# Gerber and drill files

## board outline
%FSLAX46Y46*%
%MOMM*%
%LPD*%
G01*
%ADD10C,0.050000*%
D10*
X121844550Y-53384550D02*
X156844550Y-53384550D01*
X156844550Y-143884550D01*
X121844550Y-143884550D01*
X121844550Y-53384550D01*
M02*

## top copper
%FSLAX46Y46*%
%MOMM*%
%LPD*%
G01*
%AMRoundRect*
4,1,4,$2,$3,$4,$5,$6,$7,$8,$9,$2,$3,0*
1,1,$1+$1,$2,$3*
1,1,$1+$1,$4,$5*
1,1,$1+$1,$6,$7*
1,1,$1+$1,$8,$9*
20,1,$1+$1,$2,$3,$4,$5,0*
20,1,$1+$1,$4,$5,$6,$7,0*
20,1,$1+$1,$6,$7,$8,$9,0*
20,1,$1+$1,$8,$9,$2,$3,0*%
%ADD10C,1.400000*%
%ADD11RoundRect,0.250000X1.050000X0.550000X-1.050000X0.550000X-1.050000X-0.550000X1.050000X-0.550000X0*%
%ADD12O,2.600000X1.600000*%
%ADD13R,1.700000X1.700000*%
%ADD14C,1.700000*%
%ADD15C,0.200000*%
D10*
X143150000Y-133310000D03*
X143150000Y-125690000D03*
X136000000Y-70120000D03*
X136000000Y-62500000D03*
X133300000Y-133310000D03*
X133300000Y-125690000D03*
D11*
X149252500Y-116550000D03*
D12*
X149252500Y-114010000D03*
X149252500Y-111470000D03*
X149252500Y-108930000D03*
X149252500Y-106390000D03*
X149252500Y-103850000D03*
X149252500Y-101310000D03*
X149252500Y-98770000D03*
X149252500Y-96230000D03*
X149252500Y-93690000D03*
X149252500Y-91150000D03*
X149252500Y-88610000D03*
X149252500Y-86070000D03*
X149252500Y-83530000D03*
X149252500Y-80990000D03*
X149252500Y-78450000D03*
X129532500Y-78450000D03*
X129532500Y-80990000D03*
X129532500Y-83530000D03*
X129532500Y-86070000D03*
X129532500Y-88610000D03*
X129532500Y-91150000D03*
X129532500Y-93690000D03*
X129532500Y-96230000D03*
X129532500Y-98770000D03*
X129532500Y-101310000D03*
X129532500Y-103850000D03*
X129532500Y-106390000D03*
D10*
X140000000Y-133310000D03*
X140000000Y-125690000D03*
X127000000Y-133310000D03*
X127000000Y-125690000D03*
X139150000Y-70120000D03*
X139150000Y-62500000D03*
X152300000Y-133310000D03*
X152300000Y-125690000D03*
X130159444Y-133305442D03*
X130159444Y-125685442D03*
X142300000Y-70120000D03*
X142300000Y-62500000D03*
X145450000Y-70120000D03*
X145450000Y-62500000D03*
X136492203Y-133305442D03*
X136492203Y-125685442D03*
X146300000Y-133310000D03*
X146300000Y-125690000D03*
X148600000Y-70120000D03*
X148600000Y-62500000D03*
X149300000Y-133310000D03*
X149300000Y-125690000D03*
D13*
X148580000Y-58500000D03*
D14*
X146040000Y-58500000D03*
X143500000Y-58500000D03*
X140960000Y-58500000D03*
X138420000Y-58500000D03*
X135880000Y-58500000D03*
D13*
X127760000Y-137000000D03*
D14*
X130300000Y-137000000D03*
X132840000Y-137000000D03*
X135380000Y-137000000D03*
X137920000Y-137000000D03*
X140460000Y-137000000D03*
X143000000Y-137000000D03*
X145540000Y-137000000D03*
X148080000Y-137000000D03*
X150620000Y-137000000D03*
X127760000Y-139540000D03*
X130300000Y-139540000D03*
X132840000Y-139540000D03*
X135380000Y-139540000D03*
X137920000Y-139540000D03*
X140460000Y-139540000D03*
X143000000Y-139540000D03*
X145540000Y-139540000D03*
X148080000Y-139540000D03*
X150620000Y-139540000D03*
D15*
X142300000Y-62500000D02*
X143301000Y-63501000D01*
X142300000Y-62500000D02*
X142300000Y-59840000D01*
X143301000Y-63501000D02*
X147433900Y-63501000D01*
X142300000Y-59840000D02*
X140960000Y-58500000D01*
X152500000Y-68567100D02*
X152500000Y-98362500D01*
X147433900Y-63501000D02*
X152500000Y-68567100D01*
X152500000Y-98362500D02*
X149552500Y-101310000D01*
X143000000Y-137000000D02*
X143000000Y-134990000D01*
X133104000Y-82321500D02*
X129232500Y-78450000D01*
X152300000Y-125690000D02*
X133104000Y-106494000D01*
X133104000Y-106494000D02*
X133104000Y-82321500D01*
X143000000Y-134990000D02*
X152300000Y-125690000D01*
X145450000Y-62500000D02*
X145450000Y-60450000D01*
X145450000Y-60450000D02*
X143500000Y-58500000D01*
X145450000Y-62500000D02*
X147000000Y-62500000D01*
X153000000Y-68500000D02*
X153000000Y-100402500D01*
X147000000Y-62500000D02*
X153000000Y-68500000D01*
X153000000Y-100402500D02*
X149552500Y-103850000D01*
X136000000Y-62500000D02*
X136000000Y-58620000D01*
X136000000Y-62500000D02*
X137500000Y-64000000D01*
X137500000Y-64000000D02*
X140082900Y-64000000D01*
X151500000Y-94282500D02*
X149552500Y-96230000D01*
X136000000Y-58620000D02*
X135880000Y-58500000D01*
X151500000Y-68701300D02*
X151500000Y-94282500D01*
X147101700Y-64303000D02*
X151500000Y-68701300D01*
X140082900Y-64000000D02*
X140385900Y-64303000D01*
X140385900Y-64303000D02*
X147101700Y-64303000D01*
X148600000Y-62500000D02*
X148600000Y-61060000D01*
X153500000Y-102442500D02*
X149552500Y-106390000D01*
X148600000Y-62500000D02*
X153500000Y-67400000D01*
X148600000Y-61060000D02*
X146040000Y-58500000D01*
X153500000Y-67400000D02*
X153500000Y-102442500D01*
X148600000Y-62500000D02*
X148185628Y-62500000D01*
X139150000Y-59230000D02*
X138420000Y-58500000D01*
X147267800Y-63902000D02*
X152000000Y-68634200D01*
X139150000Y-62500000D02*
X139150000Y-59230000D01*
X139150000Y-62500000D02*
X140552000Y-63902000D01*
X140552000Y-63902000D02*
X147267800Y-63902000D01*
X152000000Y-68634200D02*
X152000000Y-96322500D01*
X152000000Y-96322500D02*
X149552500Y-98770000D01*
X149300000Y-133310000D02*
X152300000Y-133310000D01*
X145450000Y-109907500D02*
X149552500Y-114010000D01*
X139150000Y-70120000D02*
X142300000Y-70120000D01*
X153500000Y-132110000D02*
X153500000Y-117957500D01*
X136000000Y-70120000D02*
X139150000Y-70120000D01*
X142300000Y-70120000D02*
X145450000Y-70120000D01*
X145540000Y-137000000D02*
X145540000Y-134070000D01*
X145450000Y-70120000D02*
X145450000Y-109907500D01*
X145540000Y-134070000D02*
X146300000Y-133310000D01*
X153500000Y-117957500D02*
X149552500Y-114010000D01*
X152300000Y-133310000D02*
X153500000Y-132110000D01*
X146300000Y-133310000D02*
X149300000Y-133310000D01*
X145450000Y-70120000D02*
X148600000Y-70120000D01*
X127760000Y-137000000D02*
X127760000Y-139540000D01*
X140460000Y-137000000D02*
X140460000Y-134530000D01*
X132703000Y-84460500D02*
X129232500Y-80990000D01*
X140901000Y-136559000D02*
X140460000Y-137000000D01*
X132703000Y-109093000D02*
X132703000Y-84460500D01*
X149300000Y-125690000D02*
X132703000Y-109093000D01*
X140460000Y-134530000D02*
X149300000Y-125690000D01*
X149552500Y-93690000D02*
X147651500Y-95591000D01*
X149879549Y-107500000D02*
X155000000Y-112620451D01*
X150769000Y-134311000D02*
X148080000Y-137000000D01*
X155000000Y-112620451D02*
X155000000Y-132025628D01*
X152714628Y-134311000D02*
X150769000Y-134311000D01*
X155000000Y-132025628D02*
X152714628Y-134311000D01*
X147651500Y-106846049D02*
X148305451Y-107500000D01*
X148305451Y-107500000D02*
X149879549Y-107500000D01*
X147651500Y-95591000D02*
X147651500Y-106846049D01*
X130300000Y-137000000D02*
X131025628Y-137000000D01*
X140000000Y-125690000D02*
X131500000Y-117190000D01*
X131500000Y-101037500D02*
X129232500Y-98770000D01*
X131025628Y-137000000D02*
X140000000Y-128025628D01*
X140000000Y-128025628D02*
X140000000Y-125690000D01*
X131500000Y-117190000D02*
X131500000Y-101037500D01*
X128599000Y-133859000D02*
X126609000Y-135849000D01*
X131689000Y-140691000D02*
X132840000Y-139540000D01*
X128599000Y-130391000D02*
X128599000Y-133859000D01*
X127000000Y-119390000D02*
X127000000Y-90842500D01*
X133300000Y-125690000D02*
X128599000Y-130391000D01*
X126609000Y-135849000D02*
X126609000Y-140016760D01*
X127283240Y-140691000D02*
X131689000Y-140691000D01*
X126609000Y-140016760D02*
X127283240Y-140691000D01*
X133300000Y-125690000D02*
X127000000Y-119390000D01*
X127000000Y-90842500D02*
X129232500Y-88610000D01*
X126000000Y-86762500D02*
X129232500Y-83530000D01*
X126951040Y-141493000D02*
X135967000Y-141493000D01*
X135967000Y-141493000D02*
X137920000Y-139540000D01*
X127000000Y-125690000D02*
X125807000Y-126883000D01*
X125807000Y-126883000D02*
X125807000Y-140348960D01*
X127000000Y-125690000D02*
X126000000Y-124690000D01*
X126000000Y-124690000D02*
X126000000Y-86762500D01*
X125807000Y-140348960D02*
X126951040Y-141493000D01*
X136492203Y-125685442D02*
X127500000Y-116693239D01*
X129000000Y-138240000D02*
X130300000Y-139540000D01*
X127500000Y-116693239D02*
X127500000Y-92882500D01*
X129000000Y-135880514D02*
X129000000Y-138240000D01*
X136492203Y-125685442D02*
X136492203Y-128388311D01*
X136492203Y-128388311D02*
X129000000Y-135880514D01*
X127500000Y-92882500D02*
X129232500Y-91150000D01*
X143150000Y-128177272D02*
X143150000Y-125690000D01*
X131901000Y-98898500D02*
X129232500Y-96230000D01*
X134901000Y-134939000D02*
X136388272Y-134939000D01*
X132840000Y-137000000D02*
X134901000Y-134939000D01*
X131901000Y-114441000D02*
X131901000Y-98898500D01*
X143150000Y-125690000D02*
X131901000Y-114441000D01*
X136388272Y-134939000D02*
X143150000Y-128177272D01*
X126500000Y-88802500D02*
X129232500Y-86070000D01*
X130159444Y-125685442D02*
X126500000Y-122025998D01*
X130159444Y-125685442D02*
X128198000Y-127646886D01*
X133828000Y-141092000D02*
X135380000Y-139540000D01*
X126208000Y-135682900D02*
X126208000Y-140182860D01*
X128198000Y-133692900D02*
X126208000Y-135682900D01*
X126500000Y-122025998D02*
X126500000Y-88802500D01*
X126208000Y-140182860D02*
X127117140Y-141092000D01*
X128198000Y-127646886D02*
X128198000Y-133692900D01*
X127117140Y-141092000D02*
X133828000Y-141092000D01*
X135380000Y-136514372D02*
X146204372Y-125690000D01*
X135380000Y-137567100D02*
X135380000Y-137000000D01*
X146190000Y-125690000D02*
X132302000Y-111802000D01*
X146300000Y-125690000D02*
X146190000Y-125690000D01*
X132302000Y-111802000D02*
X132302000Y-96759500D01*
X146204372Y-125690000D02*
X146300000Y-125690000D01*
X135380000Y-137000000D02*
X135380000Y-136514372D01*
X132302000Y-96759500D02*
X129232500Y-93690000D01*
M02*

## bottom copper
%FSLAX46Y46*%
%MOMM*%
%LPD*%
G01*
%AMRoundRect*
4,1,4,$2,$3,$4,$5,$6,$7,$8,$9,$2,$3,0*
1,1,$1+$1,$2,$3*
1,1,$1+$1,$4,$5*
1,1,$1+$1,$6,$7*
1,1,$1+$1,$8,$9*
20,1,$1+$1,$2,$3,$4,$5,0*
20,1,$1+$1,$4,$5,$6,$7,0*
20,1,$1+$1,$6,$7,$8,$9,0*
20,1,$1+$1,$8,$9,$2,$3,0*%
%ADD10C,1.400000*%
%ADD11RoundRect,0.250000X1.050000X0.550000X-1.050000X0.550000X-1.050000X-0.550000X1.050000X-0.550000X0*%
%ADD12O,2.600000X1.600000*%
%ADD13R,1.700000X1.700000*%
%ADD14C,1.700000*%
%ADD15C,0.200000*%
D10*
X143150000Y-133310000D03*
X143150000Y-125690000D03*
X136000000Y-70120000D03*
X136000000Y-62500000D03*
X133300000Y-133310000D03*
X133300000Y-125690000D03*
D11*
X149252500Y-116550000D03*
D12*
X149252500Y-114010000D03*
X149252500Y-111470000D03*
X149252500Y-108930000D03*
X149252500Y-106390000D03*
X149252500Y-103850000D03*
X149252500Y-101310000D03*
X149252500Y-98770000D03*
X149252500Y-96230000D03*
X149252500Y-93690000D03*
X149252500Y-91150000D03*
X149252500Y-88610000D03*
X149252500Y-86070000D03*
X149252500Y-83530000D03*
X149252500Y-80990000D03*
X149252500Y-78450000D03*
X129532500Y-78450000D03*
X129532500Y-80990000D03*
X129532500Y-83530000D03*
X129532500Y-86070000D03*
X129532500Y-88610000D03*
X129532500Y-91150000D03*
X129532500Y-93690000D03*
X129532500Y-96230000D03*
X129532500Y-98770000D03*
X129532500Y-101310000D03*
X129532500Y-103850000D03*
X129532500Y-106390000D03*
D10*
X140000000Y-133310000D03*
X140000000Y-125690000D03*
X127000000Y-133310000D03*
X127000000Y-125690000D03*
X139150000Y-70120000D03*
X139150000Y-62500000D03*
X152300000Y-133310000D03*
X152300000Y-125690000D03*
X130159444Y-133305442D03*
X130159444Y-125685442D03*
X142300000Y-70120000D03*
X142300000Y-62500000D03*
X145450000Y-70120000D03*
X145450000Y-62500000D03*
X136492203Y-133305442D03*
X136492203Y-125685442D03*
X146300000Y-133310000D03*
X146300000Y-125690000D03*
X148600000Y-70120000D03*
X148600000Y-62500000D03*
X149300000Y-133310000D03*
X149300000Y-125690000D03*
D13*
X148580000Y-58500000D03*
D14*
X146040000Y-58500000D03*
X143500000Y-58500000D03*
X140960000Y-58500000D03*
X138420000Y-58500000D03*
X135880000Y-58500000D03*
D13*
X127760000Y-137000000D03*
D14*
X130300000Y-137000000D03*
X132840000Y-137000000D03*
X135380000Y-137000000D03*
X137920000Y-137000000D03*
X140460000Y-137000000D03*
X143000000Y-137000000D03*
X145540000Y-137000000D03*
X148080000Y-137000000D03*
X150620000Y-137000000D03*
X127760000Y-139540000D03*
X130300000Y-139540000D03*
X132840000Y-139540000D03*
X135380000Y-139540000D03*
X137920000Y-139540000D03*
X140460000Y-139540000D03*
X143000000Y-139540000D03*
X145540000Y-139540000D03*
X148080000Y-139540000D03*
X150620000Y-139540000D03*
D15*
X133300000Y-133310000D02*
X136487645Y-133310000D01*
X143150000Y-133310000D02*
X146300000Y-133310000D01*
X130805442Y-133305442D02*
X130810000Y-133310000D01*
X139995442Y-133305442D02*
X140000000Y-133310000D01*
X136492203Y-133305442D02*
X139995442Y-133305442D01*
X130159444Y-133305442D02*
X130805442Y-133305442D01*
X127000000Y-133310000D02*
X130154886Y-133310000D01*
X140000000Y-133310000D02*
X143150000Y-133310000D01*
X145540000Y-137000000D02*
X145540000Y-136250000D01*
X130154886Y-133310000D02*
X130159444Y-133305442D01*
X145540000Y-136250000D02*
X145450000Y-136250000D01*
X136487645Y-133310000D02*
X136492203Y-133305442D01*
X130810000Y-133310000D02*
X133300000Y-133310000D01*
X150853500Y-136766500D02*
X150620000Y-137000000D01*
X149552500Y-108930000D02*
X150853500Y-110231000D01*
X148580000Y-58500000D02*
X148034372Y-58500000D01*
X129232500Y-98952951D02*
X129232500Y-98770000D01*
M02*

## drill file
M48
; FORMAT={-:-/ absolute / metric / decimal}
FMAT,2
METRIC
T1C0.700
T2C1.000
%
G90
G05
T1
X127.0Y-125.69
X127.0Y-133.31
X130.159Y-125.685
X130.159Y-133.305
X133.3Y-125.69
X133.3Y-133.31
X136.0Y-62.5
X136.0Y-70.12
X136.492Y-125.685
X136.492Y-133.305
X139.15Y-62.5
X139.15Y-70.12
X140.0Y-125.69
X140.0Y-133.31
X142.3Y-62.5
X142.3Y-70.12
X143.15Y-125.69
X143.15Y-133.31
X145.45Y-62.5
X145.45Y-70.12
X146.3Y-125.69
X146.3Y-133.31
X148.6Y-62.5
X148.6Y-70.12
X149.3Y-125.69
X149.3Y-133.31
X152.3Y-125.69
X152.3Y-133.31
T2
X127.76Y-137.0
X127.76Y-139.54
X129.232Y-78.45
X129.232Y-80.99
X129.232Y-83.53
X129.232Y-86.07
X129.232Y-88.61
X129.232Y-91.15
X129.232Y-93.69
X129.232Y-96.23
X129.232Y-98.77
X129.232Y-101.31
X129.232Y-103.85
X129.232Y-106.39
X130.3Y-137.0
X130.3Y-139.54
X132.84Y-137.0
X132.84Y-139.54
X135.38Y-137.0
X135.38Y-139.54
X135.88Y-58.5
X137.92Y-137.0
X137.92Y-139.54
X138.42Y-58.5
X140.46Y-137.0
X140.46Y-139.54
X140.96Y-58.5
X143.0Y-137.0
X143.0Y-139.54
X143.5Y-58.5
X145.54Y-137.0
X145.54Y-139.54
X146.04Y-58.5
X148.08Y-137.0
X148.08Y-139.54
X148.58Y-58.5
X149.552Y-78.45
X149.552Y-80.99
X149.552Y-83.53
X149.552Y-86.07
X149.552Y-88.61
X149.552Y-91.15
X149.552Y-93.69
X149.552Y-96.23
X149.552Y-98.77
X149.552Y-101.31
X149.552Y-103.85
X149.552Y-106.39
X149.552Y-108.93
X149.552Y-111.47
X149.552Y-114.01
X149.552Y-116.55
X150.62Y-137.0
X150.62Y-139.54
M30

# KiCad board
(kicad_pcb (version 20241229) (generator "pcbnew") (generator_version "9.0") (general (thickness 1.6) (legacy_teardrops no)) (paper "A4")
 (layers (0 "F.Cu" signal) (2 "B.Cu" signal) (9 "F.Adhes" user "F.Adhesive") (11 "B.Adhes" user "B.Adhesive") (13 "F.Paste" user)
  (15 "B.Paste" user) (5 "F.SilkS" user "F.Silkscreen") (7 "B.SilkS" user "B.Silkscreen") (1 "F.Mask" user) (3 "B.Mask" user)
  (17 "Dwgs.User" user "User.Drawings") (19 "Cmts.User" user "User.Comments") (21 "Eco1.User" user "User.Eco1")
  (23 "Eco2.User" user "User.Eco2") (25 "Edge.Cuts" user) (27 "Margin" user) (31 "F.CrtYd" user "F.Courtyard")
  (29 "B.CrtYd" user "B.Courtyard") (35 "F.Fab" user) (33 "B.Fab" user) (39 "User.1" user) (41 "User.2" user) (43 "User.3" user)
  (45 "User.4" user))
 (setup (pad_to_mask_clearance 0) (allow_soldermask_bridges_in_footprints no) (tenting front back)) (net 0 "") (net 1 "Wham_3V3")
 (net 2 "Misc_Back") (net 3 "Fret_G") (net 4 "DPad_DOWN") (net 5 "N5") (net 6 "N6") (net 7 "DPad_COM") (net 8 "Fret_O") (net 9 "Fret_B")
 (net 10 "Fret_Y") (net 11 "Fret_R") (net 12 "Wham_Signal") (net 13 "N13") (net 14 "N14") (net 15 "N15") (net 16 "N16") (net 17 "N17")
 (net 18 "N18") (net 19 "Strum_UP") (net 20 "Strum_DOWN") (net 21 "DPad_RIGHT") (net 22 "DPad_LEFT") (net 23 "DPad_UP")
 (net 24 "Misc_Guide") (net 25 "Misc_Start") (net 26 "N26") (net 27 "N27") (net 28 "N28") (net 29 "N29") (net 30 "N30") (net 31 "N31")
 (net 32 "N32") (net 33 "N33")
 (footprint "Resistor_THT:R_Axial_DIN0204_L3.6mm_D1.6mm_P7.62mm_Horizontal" (layer "F.Cu") (at 143.15 133.31 90)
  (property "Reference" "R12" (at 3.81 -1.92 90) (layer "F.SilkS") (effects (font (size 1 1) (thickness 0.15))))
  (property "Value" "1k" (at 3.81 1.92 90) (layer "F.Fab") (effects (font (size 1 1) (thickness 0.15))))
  (pad "1" thru_hole circle (at 0 0 90) (size 1.4 1.4) (drill 0.7) (layers "*.Cu" "*.Mask") (remove_unused_layers no) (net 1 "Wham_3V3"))
  (pad "2" thru_hole circle (at 7.62 0 90) (size 1.4 1.4) (drill 0.7) (layers "*.Cu" "*.Mask") (remove_unused_layers no) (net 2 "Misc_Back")))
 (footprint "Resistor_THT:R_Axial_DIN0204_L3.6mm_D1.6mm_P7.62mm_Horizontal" (layer "F.Cu") (at 136 70.12 90)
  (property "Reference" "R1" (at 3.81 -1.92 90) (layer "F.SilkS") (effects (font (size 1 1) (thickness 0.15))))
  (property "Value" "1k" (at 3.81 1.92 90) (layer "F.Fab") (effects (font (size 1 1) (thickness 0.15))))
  (pad "1" thru_hole circle (at 0 0 90) (size 1.4 1.4) (drill 0.7) (layers "*.Cu" "*.Mask") (remove_unused_layers no) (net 1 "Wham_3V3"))
  (pad "2" thru_hole circle (at 7.62 0 90) (size 1.4 1.4) (drill 0.7) (layers "*.Cu" "*.Mask") (remove_unused_layers no) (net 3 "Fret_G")))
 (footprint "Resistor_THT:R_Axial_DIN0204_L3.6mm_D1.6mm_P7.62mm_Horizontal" (layer "F.Cu") (at 133.3 133.31 90)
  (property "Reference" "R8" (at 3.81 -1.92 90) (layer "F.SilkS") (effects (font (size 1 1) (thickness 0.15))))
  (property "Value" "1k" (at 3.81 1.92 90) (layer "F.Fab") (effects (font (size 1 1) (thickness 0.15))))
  (pad "1" thru_hole circle (at 0 0 90) (size 1.4 1.4) (drill 0.7) (layers "*.Cu" "*.Mask") (remove_unused_layers no) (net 1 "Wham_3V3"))
  (pad "2" thru_hole circle (at 7.62 0 90) (size 1.4 1.4) (drill 0.7) (layers "*.Cu" "*.Mask") (remove_unused_layers no) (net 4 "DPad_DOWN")))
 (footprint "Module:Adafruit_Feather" (layer "F.Cu") (at 149.5525 116.55 180)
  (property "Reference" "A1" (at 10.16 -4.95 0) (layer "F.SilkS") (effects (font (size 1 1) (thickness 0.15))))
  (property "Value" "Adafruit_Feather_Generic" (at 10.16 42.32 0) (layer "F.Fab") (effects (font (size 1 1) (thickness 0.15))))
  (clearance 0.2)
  (pad "1" thru_hole roundrect (at 0 0 180) (size 2.6 1.6) (drill 1 (offset 0.3 0)) (layers "*.Cu" "*.Mask") (remove_unused_layers no)
   (roundrect_rratio 0.15625) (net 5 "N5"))
  (pad "2" thru_hole oval (at 0 2.54 180) (size 2.6 1.6) (drill 1 (offset 0.3 0)) (layers "*.Cu" "*.Mask") (remove_unused_layers no)
   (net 1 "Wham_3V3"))
  (pad "3" thru_hole oval (at 0 5.08 180) (size 2.6 1.6) (drill 1 (offset 0.3 0)) (layers "*.Cu" "*.Mask") (remove_unused_layers no)
   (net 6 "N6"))
  (pad "4" thru_hole oval (at 0 7.62 180) (size 2.6 1.6) (drill 1 (offset 0.3 0)) (layers "*.Cu" "*.Mask") (remove_unused_layers no)
   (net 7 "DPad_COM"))
  (pad "5" thru_hole oval (at 0 10.16 180) (size 2.6 1.6) (drill 1 (offset 0.3 0)) (layers "*.Cu" "*.Mask") (remove_unused_layers no)
   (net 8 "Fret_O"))
  (pad "6" thru_hole oval (at 0 12.7 180) (size 2.6 1.6) (drill 1 (offset 0.3 0)) (layers "*.Cu" "*.Mask") (remove_unused_layers no)
   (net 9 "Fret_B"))
  (pad "7" thru_hole oval (at 0 15.24 180) (size 2.6 1.6) (drill 1 (offset 0.3 0)) (layers "*.Cu" "*.Mask") (remove_unused_layers no)
   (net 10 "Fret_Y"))
  (pad "8" thru_hole oval (at 0 17.78 180) (size 2.6 1.6) (drill 1 (offset 0.3 0)) (layers "*.Cu" "*.Mask") (remove_unused_layers no)
   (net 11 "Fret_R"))
  (pad "9" thru_hole oval (at 0 20.32 180) (size 2.6 1.6) (drill 1 (offset 0.3 0)) (layers "*.Cu" "*.Mask") (remove_unused_layers no)
   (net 3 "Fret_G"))
  (pad "10" thru_hole oval (at 0 22.86 180) (size 2.6 1.6) (drill 1 (offset 0.3 0)) (layers "*.Cu" "*.Mask") (remove_unused_layers no)
   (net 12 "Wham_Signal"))
  (pad "11" thru_hole oval (at 0 25.4 180) (size 2.6 1.6) (drill 1 (offset 0.3 0)) (layers "*.Cu" "*.Mask") (remove_unused_layers no)
   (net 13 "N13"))
  (pad "12" thru_hole oval (at 0 27.94 180) (size 2.6 1.6) (drill 1 (offset 0.3 0)) (layers "*.Cu" "*.Mask") (remove_unused_layers no)
   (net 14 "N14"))
  (pad "13" thru_hole oval (at 0 30.48 180) (size 2.6 1.6) (drill 1 (offset 0.3 0)) (layers "*.Cu" "*.Mask") (remove_unused_layers no)
   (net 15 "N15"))
  (pad "14" thru_hole oval (at 0 33.02 180) (size 2.6 1.6) (drill 1 (offset 0.3 0)) (layers "*.Cu" "*.Mask") (remove_unused_layers no)
   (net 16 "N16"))
  (pad "15" thru_hole oval (at 0 35.56 180) (size 2.6 1.6) (drill 1 (offset 0.3 0)) (layers "*.Cu" "*.Mask") (remove_unused_layers no)
   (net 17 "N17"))
  (pad "16" thru_hole oval (at 0 38.1 180) (size 2.6 1.6) (drill 1 (offset 0.3 0)) (layers "*.Cu" "*.Mask") (remove_unused_layers no)
   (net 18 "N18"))
  (pad "17" thru_hole oval (at 20.32 38.1) (size 2.6 1.6) (drill 1 (offset 0.3 0)) (layers "*.Cu" "*.Mask") (remove_unused_layers no)
   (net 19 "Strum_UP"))
  (pad "18" thru_hole oval (at 20.32 35.56) (size 2.6 1.6) (drill 1 (offset 0.3 0)) (layers "*.Cu" "*.Mask") (remove_unused_layers no)
   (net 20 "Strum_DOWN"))
  (pad "19" thru_hole oval (at 20.32 33.02) (size 2.6 1.6) (drill 1 (offset 0.3 0)) (layers "*.Cu" "*.Mask") (remove_unused_layers no)
   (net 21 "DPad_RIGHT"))
  (pad "20" thru_hole oval (at 20.32 30.48) (size 2.6 1.6) (drill 1 (offset 0.3 0)) (layers "*.Cu" "*.Mask") (remove_unused_layers no)
   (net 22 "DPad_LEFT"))
  (pad "21" thru_hole oval (at 20.32 27.94) (size 2.6 1.6) (drill 1 (offset 0.3 0)) (layers "*.Cu" "*.Mask") (remove_unused_layers no)
   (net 4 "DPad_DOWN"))
  (pad "22" thru_hole oval (at 20.32 25.4) (size 2.6 1.6) (drill 1 (offset 0.3 0)) (layers "*.Cu" "*.Mask") (remove_unused_layers no)
   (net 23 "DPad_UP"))
  (pad "23" thru_hole oval (at 20.32 22.86) (size 2.6 1.6) (drill 1 (offset 0.3 0)) (layers "*.Cu" "*.Mask") (remove_unused_layers no)
   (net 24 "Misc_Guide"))
  (pad "24" thru_hole oval (at 20.32 20.32) (size 2.6 1.6) (drill 1 (offset 0.3 0)) (layers "*.Cu" "*.Mask") (remove_unused_layers no)
   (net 2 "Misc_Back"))
  (pad "25" thru_hole oval (at 20.32 17.78) (size 2.6 1.6) (drill 1 (offset 0.3 0)) (layers "*.Cu" "*.Mask") (remove_unused_layers no)
   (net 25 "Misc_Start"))
  (pad "26" thru_hole oval (at 20.32 15.24) (size 2.6 1.6) (drill 1 (offset 0.3 0)) (layers "*.Cu" "*.Mask") (remove_unused_layers no)
   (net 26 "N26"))
  (pad "27" thru_hole oval (at 20.32 12.7) (size 2.6 1.6) (drill 1 (offset 0.3 0)) (layers "*.Cu" "*.Mask") (remove_unused_layers no)
   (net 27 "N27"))
  (pad "28" thru_hole oval (at 20.32 10.16) (size 2.6 1.6) (drill 1 (offset 0.3 0)) (layers "*.Cu" "*.Mask") (remove_unused_layers no)
   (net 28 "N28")))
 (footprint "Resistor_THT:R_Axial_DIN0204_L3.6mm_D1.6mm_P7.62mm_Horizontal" (layer "F.Cu") (at 140 133.31 90)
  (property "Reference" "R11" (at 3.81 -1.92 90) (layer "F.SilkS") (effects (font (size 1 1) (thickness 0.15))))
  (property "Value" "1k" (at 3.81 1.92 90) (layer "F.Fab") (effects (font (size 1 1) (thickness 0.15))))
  (pad "1" thru_hole circle (at 0 0 90) (size 1.4 1.4) (drill 0.7) (layers "*.Cu" "*.Mask") (remove_unused_layers no) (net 1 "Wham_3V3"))
  (pad "2" thru_hole circle (at 7.62 0 90) (size 1.4 1.4) (drill 0.7) (layers "*.Cu" "*.Mask") (remove_unused_layers no)
   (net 25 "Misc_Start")))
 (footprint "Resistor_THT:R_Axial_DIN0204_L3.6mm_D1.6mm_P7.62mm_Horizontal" (layer "F.Cu") (at 127 133.31 90)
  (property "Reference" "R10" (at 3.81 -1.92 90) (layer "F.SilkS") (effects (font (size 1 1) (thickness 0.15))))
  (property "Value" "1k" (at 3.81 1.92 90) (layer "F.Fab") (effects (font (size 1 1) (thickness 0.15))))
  (pad "1" thru_hole circle (at 0 0 90) (size 1.4 1.4) (drill 0.7) (layers "*.Cu" "*.Mask") (remove_unused_layers no) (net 1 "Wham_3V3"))
  (pad "2" thru_hole circle (at 7.62 0 90) (size 1.4 1.4) (drill 0.7) (layers "*.Cu" "*.Mask") (remove_unused_layers no)
   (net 21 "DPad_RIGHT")))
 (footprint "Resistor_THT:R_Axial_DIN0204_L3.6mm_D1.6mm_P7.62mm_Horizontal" (layer "F.Cu") (at 139.15 70.12 90)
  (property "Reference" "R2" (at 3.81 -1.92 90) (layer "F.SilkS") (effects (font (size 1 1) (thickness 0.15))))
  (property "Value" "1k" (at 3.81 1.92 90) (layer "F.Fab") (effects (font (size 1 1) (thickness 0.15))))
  (pad "1" thru_hole circle (at 0 0 90) (size 1.4 1.4) (drill 0.7) (layers "*.Cu" "*.Mask") (remove_unused_layers no) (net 1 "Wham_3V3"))
  (pad "2" thru_hole circle (at 7.62 0 90) (size 1.4 1.4) (drill 0.7) (layers "*.Cu" "*.Mask") (remove_unused_layers no) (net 11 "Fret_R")))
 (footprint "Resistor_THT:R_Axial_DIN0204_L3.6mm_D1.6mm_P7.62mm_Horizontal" (layer "F.Cu") (at 152.3 133.31 90)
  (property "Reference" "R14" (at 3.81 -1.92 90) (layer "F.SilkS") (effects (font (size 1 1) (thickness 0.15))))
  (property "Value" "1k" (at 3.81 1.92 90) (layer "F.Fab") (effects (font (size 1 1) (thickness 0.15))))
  (pad "1" thru_hole circle (at 0 0 90) (size 1.4 1.4) (drill 0.7) (layers "*.Cu" "*.Mask") (remove_unused_layers no) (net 1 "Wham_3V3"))
  (pad "2" thru_hole circle (at 7.62 0 90) (size 1.4 1.4) (drill 0.7) (layers "*.Cu" "*.Mask") (remove_unused_layers no) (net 19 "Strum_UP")))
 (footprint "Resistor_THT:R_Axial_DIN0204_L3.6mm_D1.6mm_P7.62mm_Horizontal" (layer "F.Cu") (at 130.159444 133.305442 90)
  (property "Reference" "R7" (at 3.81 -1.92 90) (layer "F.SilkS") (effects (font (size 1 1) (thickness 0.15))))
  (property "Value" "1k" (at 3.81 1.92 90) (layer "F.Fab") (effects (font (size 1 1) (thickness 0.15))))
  (pad "1" thru_hole circle (at 0 0 90) (size 1.4 1.4) (drill 0.7) (layers "*.Cu" "*.Mask") (remove_unused_layers no) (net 1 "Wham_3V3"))
  (pad "2" thru_hole circle (at 7.62 0 90) (size 1.4 1.4) (drill 0.7) (layers "*.Cu" "*.Mask") (remove_unused_layers no)
   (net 22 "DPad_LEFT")))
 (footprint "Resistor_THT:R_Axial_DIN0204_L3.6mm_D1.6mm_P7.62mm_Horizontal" (layer "F.Cu") (at 142.3 70.12 90)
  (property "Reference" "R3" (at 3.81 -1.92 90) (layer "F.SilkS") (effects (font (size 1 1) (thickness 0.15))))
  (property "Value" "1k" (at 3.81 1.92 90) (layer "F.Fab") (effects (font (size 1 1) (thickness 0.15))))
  (pad "1" thru_hole circle (at 0 0 90) (size 1.4 1.4) (drill 0.7) (layers "*.Cu" "*.Mask") (remove_unused_layers no) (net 1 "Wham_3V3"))
  (pad "2" thru_hole circle (at 7.62 0 90) (size 1.4 1.4) (drill 0.7) (layers "*.Cu" "*.Mask") (remove_unused_layers no) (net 10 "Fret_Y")))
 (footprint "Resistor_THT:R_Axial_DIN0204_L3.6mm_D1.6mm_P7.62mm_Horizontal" (layer "F.Cu") (at 145.45 70.12 90)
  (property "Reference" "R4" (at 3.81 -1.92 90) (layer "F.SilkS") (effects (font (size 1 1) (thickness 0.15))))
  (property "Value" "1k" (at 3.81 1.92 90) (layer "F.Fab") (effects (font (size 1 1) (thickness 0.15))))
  (pad "1" thru_hole circle (at 0 0 90) (size 1.4 1.4) (drill 0.7) (layers "*.Cu" "*.Mask") (remove_unused_layers no) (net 1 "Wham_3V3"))
  (pad "2" thru_hole circle (at 7.62 0 90) (size 1.4 1.4) (drill 0.7) (layers "*.Cu" "*.Mask") (remove_unused_layers no) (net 9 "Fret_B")))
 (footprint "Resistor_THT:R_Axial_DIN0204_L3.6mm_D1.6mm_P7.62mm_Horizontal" (layer "F.Cu") (at 136.492203 133.305442 90)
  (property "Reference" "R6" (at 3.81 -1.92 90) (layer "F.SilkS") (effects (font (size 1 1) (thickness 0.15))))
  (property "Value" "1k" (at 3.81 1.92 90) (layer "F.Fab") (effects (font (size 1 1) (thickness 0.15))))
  (pad "1" thru_hole circle (at 0 0 90) (size 1.4 1.4) (drill 0.7) (layers "*.Cu" "*.Mask") (remove_unused_layers no) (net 1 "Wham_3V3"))
  (pad "2" thru_hole circle (at 7.62 0 90) (size 1.4 1.4) (drill 0.7) (layers "*.Cu" "*.Mask") (remove_unused_layers no) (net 23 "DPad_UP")))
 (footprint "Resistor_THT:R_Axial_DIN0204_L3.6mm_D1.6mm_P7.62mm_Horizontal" (layer "F.Cu") (at 146.3 133.31 90)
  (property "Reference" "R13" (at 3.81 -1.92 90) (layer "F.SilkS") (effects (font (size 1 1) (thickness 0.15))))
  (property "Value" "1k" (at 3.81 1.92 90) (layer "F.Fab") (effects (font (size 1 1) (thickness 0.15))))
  (pad "1" thru_hole circle (at 0 0 90) (size 1.4 1.4) (drill 0.7) (layers "*.Cu" "*.Mask") (remove_unused_layers no) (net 1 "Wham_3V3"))
  (pad "2" thru_hole circle (at 7.62 0 90) (size 1.4 1.4) (drill 0.7) (layers "*.Cu" "*.Mask") (remove_unused_layers no)
   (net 24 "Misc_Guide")))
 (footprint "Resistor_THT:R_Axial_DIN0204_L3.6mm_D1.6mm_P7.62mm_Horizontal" (layer "F.Cu") (at 148.6 70.12 90)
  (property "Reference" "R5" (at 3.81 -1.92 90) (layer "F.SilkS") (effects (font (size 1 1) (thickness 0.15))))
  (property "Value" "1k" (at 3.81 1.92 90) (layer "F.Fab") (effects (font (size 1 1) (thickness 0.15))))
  (pad "1" thru_hole circle (at 0 0 90) (size 1.4 1.4) (drill 0.7) (layers "*.Cu" "*.Mask") (remove_unused_layers no) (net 1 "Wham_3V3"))
  (pad "2" thru_hole circle (at 7.62 0 90) (size 1.4 1.4) (drill 0.7) (layers "*.Cu" "*.Mask") (remove_unused_layers no) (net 8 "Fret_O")))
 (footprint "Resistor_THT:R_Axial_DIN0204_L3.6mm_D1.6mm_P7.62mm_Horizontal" (layer "F.Cu") (at 149.3 133.31 90)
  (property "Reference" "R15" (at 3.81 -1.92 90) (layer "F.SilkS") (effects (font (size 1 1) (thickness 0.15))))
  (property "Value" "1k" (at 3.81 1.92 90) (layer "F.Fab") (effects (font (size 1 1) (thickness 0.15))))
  (pad "1" thru_hole circle (at 0 0 90) (size 1.4 1.4) (drill 0.7) (layers "*.Cu" "*.Mask") (remove_unused_layers no) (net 1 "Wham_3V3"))
  (pad "2" thru_hole circle (at 7.62 0 90) (size 1.4 1.4) (drill 0.7) (layers "*.Cu" "*.Mask") (remove_unused_layers no)
   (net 20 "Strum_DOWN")))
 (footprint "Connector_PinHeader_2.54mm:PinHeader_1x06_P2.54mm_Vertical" (layer "B.Cu") (at 148.58 58.5 90)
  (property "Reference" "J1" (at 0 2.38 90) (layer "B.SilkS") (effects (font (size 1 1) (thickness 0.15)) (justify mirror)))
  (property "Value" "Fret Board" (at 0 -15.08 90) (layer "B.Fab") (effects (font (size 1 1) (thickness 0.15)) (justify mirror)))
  (pad "1" thru_hole rect (at 0 0 90) (size 1.7 1.7) (drill 1) (layers "*.Cu" "*.Mask") (remove_unused_layers no) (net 7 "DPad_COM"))
  (pad "2" thru_hole circle (at 0 -2.54 90) (size 1.7 1.7) (drill 1) (layers "*.Cu" "*.Mask") (remove_unused_layers no) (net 8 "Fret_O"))
  (pad "3" thru_hole circle (at 0 -5.08 90) (size 1.7 1.7) (drill 1) (layers "*.Cu" "*.Mask") (remove_unused_layers no) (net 9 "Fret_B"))
  (pad "4" thru_hole circle (at 0 -7.62 90) (size 1.7 1.7) (drill 1) (layers "*.Cu" "*.Mask") (remove_unused_layers no) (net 10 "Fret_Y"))
  (pad "5" thru_hole circle (at 0 -10.16 90) (size 1.7 1.7) (drill 1) (layers "*.Cu" "*.Mask") (remove_unused_layers no) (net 11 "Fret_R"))
  (pad "6" thru_hole circle (at 0 -12.7 90) (size 1.7 1.7) (drill 1) (layers "*.Cu" "*.Mask") (remove_unused_layers no) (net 3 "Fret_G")))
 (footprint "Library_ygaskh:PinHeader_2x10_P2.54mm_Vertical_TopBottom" (layer "B.Cu") (at 127.76 137 -90)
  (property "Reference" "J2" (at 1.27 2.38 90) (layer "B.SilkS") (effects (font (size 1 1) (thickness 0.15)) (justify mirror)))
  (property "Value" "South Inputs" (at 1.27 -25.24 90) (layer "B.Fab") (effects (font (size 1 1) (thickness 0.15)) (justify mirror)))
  (pad "1" thru_hole rect (at 0 0 270) (size 1.7 1.7) (drill 1) (layers "*.Cu" "*.Mask") (remove_unused_layers no) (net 7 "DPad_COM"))
  (pad "2" thru_hole circle (at 0 -2.54 270) (size 1.7 1.7) (drill 1) (layers "*.Cu" "*.Mask") (remove_unused_layers no)
   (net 25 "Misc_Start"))
  (pad "3" thru_hole circle (at 0 -5.08 270) (size 1.7 1.7) (drill 1) (layers "*.Cu" "*.Mask") (remove_unused_layers no) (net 2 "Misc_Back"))
  (pad "4" thru_hole circle (at 0 -7.62 270) (size 1.7 1.7) (drill 1) (layers "*.Cu" "*.Mask") (remove_unused_layers no)
   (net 24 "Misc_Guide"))
  (pad "5" thru_hole circle (at 0 -10.16 270) (size 1.7 1.7) (drill 1) (layers "*.Cu" "*.Mask") (remove_unused_layers no) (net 7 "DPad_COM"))
  (pad "6" thru_hole circle (at 0 -12.7 270) (size 1.7 1.7) (drill 1) (layers "*.Cu" "*.Mask") (remove_unused_layers no)
   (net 20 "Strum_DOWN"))
  (pad "7" thru_hole circle (at 0 -15.24 270) (size 1.7 1.7) (drill 1) (layers "*.Cu" "*.Mask") (remove_unused_layers no)
   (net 19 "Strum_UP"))
  (pad "8" thru_hole circle (at 0 -17.78 270) (size 1.7 1.7) (drill 1) (layers "*.Cu" "*.Mask") (remove_unused_layers no) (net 1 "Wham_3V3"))
  (pad "9" thru_hole circle (at 0 -20.32 270) (size 1.7 1.7) (drill 1) (layers "*.Cu" "*.Mask") (remove_unused_layers no)
   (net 12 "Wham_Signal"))
  (pad "10" thru_hole circle (at 0 -22.86 270) (size 1.7 1.7) (drill 1) (layers "*.Cu" "*.Mask") (remove_unused_layers no)
   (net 7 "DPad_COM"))
  (pad "11" thru_hole circle (at 2.54 0 270) (size 1.7 1.7) (drill 1) (layers "*.Cu" "*.Mask") (remove_unused_layers no) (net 7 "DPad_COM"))
  (pad "12" thru_hole circle (at 2.54 -2.54 270) (size 1.7 1.7) (drill 1) (layers "*.Cu" "*.Mask") (remove_unused_layers no)
   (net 23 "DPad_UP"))
  (pad "13" thru_hole circle (at 2.54 -5.08 270) (size 1.7 1.7) (drill 1) (layers "*.Cu" "*.Mask") (remove_unused_layers no)
   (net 4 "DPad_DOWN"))
  (pad "14" thru_hole circle (at 2.54 -7.62 270) (size 1.7 1.7) (drill 1) (layers "*.Cu" "*.Mask") (remove_unused_layers no)
   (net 22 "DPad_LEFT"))
  (pad "15" thru_hole circle (at 2.54 -10.16 270) (size 1.7 1.7) (drill 1) (layers "*.Cu" "*.Mask") (remove_unused_layers no)
   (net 21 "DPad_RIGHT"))
  (pad "16" thru_hole circle (at 2.54 -12.7 270) (size 1.7 1.7) (drill 1) (layers "*.Cu" "*.Mask") (remove_unused_layers no) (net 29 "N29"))
  (pad "17" thru_hole circle (at 2.54 -15.24 270) (size 1.7 1.7) (drill 1) (layers "*.Cu" "*.Mask") (remove_unused_layers no) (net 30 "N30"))
  (pad "18" thru_hole circle (at 2.54 -17.78 270) (size 1.7 1.7) (drill 1) (layers "*.Cu" "*.Mask") (remove_unused_layers no) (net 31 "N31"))
  (pad "19" thru_hole circle (at 2.54 -20.32 270) (size 1.7 1.7) (drill 1) (layers "*.Cu" "*.Mask") (remove_unused_layers no) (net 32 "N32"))
  (pad "20" thru_hole circle (at 2.54 -22.86 270) (size 1.7 1.7) (drill 1) (layers "*.Cu" "*.Mask") (remove_unused_layers no) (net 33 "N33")))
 (gr_rect (start 121.84455 53.38455) (end 156.84455 143.88455) (stroke (width 0.05) (type default)) (fill no) (layer "Edge.Cuts"))
 (segment (start 142.3 62.5) (end 143.301 63.501) (width 0.2) (layer "F.Cu") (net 10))
 (segment (start 142.3 62.5) (end 142.3 59.84) (width 0.2) (layer "F.Cu") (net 10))
 (segment (start 143.301 63.501) (end 147.4339 63.501) (width 0.2) (layer "F.Cu") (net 10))
 (segment (start 142.3 59.84) (end 140.96 58.5) (width 0.2) (layer "F.Cu") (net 10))
 (segment (start 152.5 68.5671) (end 152.5 98.3625) (width 0.2) (layer "F.Cu") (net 10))
 (segment (start 147.4339 63.501) (end 152.5 68.5671) (width 0.2) (layer "F.Cu") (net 10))
 (segment (start 152.5 98.3625) (end 149.5525 101.31) (width 0.2) (layer "F.Cu") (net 10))
 (segment (start 143 137) (end 143 134.99) (width 0.2) (layer "F.Cu") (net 19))
 (segment (start 133.104 82.3215) (end 129.2325 78.45) (width 0.2) (layer "F.Cu") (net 19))
 (segment (start 152.3 125.69) (end 133.104 106.494) (width 0.2) (layer "F.Cu") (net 19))
 (segment (start 133.104 106.494) (end 133.104 82.3215) (width 0.2) (layer "F.Cu") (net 19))
 (segment (start 143 134.99) (end 152.3 125.69) (width 0.2) (layer "F.Cu") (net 19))
 (segment (start 145.45 62.5) (end 145.45 60.45) (width 0.2) (layer "F.Cu") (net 9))
 (segment (start 145.45 60.45) (end 143.5 58.5) (width 0.2) (layer "F.Cu") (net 9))
 (segment (start 145.45 62.5) (end 147 62.5) (width 0.2) (layer "F.Cu") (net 9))
 (segment (start 153 68.5) (end 153 100.4025) (width 0.2) (layer "F.Cu") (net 9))
 (segment (start 147 62.5) (end 153 68.5) (width 0.2) (layer "F.Cu") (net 9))
 (segment (start 153 100.4025) (end 149.5525 103.85) (width 0.2) (layer "F.Cu") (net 9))
 (segment (start 136 62.5) (end 136 58.62) (width 0.2) (layer "F.Cu") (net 3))
 (segment (start 136 62.5) (end 137.5 64) (width 0.2) (layer "F.Cu") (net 3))
 (segment (start 137.5 64) (end 140.0829 64) (width 0.2) (layer "F.Cu") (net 3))
 (segment (start 151.5 94.2825) (end 149.5525 96.23) (width 0.2) (layer "F.Cu") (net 3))
 (segment (start 136 58.62) (end 135.88 58.5) (width 0.2) (layer "F.Cu") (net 3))
 (segment (start 151.5 68.7013) (end 151.5 94.2825) (width 0.2) (layer "F.Cu") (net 3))
 (segment (start 147.1017 64.303) (end 151.5 68.7013) (width 0.2) (layer "F.Cu") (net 3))
 (segment (start 140.0829 64) (end 140.3859 64.303) (width 0.2) (layer "F.Cu") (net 3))
 (segment (start 140.3859 64.303) (end 147.1017 64.303) (width 0.2) (layer "F.Cu") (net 3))
 (segment (start 148.6 62.5) (end 148.6 61.06) (width 0.2) (layer "F.Cu") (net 8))
 (segment (start 153.5 102.4425) (end 149.5525 106.39) (width 0.2) (layer "F.Cu") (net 8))
 (segment (start 148.6 62.5) (end 153.5 67.4) (width 0.2) (layer "F.Cu") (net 8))
 (segment (start 148.6 61.06) (end 146.04 58.5) (width 0.2) (layer "F.Cu") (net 8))
 (segment (start 153.5 67.4) (end 153.5 102.4425) (width 0.2) (layer "F.Cu") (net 8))
 (segment (start 148.6 62.5) (end 148.185628 62.5) (width 0.2) (layer "F.Cu") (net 8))
 (segment (start 139.15 59.23) (end 138.42 58.5) (width 0.2) (layer "F.Cu") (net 11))
 (segment (start 147.2678 63.902) (end 152 68.6342) (width 0.2) (layer "F.Cu") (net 11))
 (segment (start 139.15 62.5) (end 139.15 59.23) (width 0.2) (layer "F.Cu") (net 11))
 (segment (start 139.15 62.5) (end 140.552 63.902) (width 0.2) (layer "F.Cu") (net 11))
 (segment (start 140.552 63.902) (end 147.2678 63.902) (width 0.2) (layer "F.Cu") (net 11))
 (segment (start 152 68.6342) (end 152 96.3225) (width 0.2) (layer "F.Cu") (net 11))
 (segment (start 152 96.3225) (end 149.5525 98.77) (width 0.2) (layer "F.Cu") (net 11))
 (segment (start 149.3 133.31) (end 152.3 133.31) (width 0.2) (layer "F.Cu") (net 1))
 (segment (start 145.45 109.9075) (end 149.5525 114.01) (width 0.2) (layer "F.Cu") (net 1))
 (segment (start 139.15 70.12) (end 142.3 70.12) (width 0.2) (layer "F.Cu") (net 1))
 (segment (start 153.5 132.11) (end 153.5 117.9575) (width 0.2) (layer "F.Cu") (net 1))
 (segment (start 136 70.12) (end 139.15 70.12) (width 0.2) (layer "F.Cu") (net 1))
 (segment (start 142.3 70.12) (end 145.45 70.12) (width 0.2) (layer "F.Cu") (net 1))
 (segment (start 145.54 137) (end 145.54 134.07) (width 0.2) (layer "F.Cu") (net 1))
 (segment (start 145.45 70.12) (end 145.45 109.9075) (width 0.2) (layer "F.Cu") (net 1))
 (segment (start 145.54 134.07) (end 146.3 133.31) (width 0.2) (layer "F.Cu") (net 1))
 (segment (start 153.5 117.9575) (end 149.5525 114.01) (width 0.2) (layer "F.Cu") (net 1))
 (segment (start 152.3 133.31) (end 153.5 132.11) (width 0.2) (layer "F.Cu") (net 1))
 (segment (start 146.3 133.31) (end 149.3 133.31) (width 0.2) (layer "F.Cu") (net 1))
 (segment (start 145.45 70.12) (end 148.6 70.12) (width 0.2) (layer "F.Cu") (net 1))
 (segment (start 133.3 133.31) (end 136.487645 133.31) (width 0.2) (layer "B.Cu") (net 1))
 (segment (start 143.15 133.31) (end 146.3 133.31) (width 0.2) (layer "B.Cu") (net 1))
 (segment (start 130.805442 133.305442) (end 130.81 133.31) (width 0.2) (layer "B.Cu") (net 1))
 (segment (start 139.995442 133.305442) (end 140 133.31) (width 0.2) (layer "B.Cu") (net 1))
 (segment (start 136.492203 133.305442) (end 139.995442 133.305442) (width 0.2) (layer "B.Cu") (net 1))
 (segment (start 130.159444 133.305442) (end 130.805442 133.305442) (width 0.2) (layer "B.Cu") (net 1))
 (segment (start 127 133.31) (end 130.154886 133.31) (width 0.2) (layer "B.Cu") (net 1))
 (segment (start 140 133.31) (end 143.15 133.31) (width 0.2) (layer "B.Cu") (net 1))
 (segment (start 145.54 137) (end 145.54 136.25) (width 0.2) (layer "B.Cu") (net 1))
 (segment (start 130.154886 133.31) (end 130.159444 133.305442) (width 0.2) (layer "B.Cu") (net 1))
 (segment (start 145.54 136.25) (end 145.45 136.25) (width 0.2) (layer "B.Cu") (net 1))
 (segment (start 136.487645 133.31) (end 136.492203 133.305442) (width 0.2) (layer "B.Cu") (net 1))
 (segment (start 130.81 133.31) (end 133.3 133.31) (width 0.2) (layer "B.Cu") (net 1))
 (segment (start 127.76 137) (end 127.76 139.54) (width 0.2) (layer "F.Cu") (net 7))
 (segment (start 150.8535 136.7665) (end 150.62 137) (width 0.2) (layer "B.Cu") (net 7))
 (segment (start 149.5525 108.93) (end 150.8535 110.231) (width 0.2) (layer "B.Cu") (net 7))
 (segment (start 148.58 58.5) (end 148.034372 58.5) (width 0.2) (layer "B.Cu") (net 7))
 (segment (start 140.46 137) (end 140.46 134.53) (width 0.2) (layer "F.Cu") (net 20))
 (segment (start 132.703 84.4605) (end 129.2325 80.99) (width 0.2) (layer "F.Cu") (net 20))
 (segment (start 140.901 136.559) (end 140.46 137) (width 0.2) (layer "F.Cu") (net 20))
 (segment (start 132.703 109.093) (end 132.703 84.4605) (width 0.2) (layer "F.Cu") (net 20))
 (segment (start 149.3 125.69) (end 132.703 109.093) (width 0.2) (layer "F.Cu") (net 20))
 (segment (start 140.46 134.53) (end 149.3 125.69) (width 0.2) (layer "F.Cu") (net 20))
 (segment (start 149.5525 93.69) (end 147.6515 95.591) (width 0.2) (layer "F.Cu") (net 12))
 (segment (start 149.879549 107.5) (end 155 112.620451) (width 0.2) (layer "F.Cu") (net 12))
 (segment (start 150.769 134.311) (end 148.08 137) (width 0.2) (layer "F.Cu") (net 12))
 (segment (start 155 112.620451) (end 155 132.025628) (width 0.2) (layer "F.Cu") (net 12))
 (segment (start 152.714628 134.311) (end 150.769 134.311) (width 0.2) (layer "F.Cu") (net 12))
 (segment (start 155 132.025628) (end 152.714628 134.311) (width 0.2) (layer "F.Cu") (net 12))
 (segment (start 147.6515 106.846049) (end 148.305451 107.5) (width 0.2) (layer "F.Cu") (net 12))
 (segment (start 148.305451 107.5) (end 149.879549 107.5) (width 0.2) (layer "F.Cu") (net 12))
 (segment (start 147.6515 95.591) (end 147.6515 106.846049) (width 0.2) (layer "F.Cu") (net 12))
 (segment (start 130.3 137) (end 131.025628 137) (width 0.2) (layer "F.Cu") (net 25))
 (segment (start 140 125.69) (end 131.5 117.19) (width 0.2) (layer "F.Cu") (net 25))
 (segment (start 131.5 101.0375) (end 129.2325 98.77) (width 0.2) (layer "F.Cu") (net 25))
 (segment (start 131.025628 137) (end 140 128.025628) (width 0.2) (layer "F.Cu") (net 25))
 (segment (start 140 128.025628) (end 140 125.69) (width 0.2) (layer "F.Cu") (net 25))
 (segment (start 131.5 117.19) (end 131.5 101.0375) (width 0.2) (layer "F.Cu") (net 25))
 (segment (start 129.2325 98.952951) (end 129.2325 98.77) (width 0.2) (layer "B.Cu") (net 25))
 (segment (start 128.599 133.859) (end 126.609 135.849) (width 0.2) (layer "F.Cu") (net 4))
 (segment (start 131.689 140.691) (end 132.84 139.54) (width 0.2) (layer "F.Cu") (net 4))
 (segment (start 128.599 130.391) (end 128.599 133.859) (width 0.2) (layer "F.Cu") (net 4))
 (segment (start 127 119.39) (end 127 90.8425) (width 0.2) (layer "F.Cu") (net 4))
 (segment (start 133.3 125.69) (end 128.599 130.391) (width 0.2) (layer "F.Cu") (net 4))
 (segment (start 126.609 135.849) (end 126.609 140.01676) (width 0.2) (layer "F.Cu") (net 4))
 (segment (start 127.28324 140.691) (end 131.689 140.691) (width 0.2) (layer "F.Cu") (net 4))
 (segment (start 126.609 140.01676) (end 127.28324 140.691) (width 0.2) (layer "F.Cu") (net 4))
 (segment (start 133.3 125.69) (end 127 119.39) (width 0.2) (layer "F.Cu") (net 4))
 (segment (start 127 90.8425) (end 129.2325 88.61) (width 0.2) (layer "F.Cu") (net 4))
 (segment (start 126 86.7625) (end 129.2325 83.53) (width 0.2) (layer "F.Cu") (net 21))
 (segment (start 126.95104 141.493) (end 135.967 141.493) (width 0.2) (layer "F.Cu") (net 21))
 (segment (start 135.967 141.493) (end 137.92 139.54) (width 0.2) (layer "F.Cu") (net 21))
 (segment (start 127 125.69) (end 125.807 126.883) (width 0.2) (layer "F.Cu") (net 21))
 (segment (start 125.807 126.883) (end 125.807 140.34896) (width 0.2) (layer "F.Cu") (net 21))
 (segment (start 127 125.69) (end 126 124.69) (width 0.2) (layer "F.Cu") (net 21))
 (segment (start 126 124.69) (end 126 86.7625) (width 0.2) (layer "F.Cu") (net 21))
 (segment (start 125.807 140.34896) (end 126.95104 141.493) (width 0.2) (layer "F.Cu") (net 21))
 (segment (start 136.492203 125.685442) (end 127.5 116.693239) (width 0.2) (layer "F.Cu") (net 23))
 (segment (start 129 138.24) (end 130.3 139.54) (width 0.2) (layer "F.Cu") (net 23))
 (segment (start 127.5 116.693239) (end 127.5 92.8825) (width 0.2) (layer "F.Cu") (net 23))
 (segment (start 129 135.880514) (end 129 138.24) (width 0.2) (layer "F.Cu") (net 23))
 (segment (start 136.492203 125.685442) (end 136.492203 128.388311) (width 0.2) (layer "F.Cu") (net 23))
 (segment (start 136.492203 128.388311) (end 129 135.880514) (width 0.2) (layer "F.Cu") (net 23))
 (segment (start 127.5 92.8825) (end 129.2325 91.15) (width 0.2) (layer "F.Cu") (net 23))
 (segment (start 143.15 128.177272) (end 143.15 125.69) (width 0.2) (layer "F.Cu") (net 2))
 (segment (start 131.901 98.8985) (end 129.2325 96.23) (width 0.2) (layer "F.Cu") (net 2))
 (segment (start 134.901 134.939) (end 136.388272 134.939) (width 0.2) (layer "F.Cu") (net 2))
 (segment (start 132.84 137) (end 134.901 134.939) (width 0.2) (layer "F.Cu") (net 2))
 (segment (start 131.901 114.441) (end 131.901 98.8985) (width 0.2) (layer "F.Cu") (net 2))
 (segment (start 143.15 125.69) (end 131.901 114.441) (width 0.2) (layer "F.Cu") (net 2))
 (segment (start 136.388272 134.939) (end 143.15 128.177272) (width 0.2) (layer "F.Cu") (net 2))
 (segment (start 126.5 88.8025) (end 129.2325 86.07) (width 0.2) (layer "F.Cu") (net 22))
 (segment (start 130.159444 125.685442) (end 126.5 122.025998) (width 0.2) (layer "F.Cu") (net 22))
 (segment (start 130.159444 125.685442) (end 128.198 127.646886) (width 0.2) (layer "F.Cu") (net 22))
 (segment (start 133.828 141.092) (end 135.38 139.54) (width 0.2) (layer "F.Cu") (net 22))
 (segment (start 126.208 135.6829) (end 126.208 140.18286) (width 0.2) (layer "F.Cu") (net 22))
 (segment (start 128.198 133.6929) (end 126.208 135.6829) (width 0.2) (layer "F.Cu") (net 22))
 (segment (start 126.5 122.025998) (end 126.5 88.8025) (width 0.2) (layer "F.Cu") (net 22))
 (segment (start 126.208 140.18286) (end 127.11714 141.092) (width 0.2) (layer "F.Cu") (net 22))
 (segment (start 128.198 127.646886) (end 128.198 133.6929) (width 0.2) (layer "F.Cu") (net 22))
 (segment (start 127.11714 141.092) (end 133.828 141.092) (width 0.2) (layer "F.Cu") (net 22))
 (segment (start 135.38 136.514372) (end 146.204372 125.69) (width 0.2) (layer "F.Cu") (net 24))
 (segment (start 135.38 137.5671) (end 135.38 137) (width 0.2) (layer "F.Cu") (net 24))
 (segment (start 146.19 125.69) (end 132.302 111.802) (width 0.2) (layer "F.Cu") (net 24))
 (segment (start 146.3 125.69) (end 146.19 125.69) (width 0.2) (layer "F.Cu") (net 24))
 (segment (start 132.302 111.802) (end 132.302 96.7595) (width 0.2) (layer "F.Cu") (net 24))
 (segment (start 146.204372 125.69) (end 146.3 125.69) (width 0.2) (layer "F.Cu") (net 24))
 (segment (start 135.38 137) (end 135.38 136.514372) (width 0.2) (layer "F.Cu") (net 24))
 (segment (start 132.302 96.7595) (end 129.2325 93.69) (width 0.2) (layer "F.Cu") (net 24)))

